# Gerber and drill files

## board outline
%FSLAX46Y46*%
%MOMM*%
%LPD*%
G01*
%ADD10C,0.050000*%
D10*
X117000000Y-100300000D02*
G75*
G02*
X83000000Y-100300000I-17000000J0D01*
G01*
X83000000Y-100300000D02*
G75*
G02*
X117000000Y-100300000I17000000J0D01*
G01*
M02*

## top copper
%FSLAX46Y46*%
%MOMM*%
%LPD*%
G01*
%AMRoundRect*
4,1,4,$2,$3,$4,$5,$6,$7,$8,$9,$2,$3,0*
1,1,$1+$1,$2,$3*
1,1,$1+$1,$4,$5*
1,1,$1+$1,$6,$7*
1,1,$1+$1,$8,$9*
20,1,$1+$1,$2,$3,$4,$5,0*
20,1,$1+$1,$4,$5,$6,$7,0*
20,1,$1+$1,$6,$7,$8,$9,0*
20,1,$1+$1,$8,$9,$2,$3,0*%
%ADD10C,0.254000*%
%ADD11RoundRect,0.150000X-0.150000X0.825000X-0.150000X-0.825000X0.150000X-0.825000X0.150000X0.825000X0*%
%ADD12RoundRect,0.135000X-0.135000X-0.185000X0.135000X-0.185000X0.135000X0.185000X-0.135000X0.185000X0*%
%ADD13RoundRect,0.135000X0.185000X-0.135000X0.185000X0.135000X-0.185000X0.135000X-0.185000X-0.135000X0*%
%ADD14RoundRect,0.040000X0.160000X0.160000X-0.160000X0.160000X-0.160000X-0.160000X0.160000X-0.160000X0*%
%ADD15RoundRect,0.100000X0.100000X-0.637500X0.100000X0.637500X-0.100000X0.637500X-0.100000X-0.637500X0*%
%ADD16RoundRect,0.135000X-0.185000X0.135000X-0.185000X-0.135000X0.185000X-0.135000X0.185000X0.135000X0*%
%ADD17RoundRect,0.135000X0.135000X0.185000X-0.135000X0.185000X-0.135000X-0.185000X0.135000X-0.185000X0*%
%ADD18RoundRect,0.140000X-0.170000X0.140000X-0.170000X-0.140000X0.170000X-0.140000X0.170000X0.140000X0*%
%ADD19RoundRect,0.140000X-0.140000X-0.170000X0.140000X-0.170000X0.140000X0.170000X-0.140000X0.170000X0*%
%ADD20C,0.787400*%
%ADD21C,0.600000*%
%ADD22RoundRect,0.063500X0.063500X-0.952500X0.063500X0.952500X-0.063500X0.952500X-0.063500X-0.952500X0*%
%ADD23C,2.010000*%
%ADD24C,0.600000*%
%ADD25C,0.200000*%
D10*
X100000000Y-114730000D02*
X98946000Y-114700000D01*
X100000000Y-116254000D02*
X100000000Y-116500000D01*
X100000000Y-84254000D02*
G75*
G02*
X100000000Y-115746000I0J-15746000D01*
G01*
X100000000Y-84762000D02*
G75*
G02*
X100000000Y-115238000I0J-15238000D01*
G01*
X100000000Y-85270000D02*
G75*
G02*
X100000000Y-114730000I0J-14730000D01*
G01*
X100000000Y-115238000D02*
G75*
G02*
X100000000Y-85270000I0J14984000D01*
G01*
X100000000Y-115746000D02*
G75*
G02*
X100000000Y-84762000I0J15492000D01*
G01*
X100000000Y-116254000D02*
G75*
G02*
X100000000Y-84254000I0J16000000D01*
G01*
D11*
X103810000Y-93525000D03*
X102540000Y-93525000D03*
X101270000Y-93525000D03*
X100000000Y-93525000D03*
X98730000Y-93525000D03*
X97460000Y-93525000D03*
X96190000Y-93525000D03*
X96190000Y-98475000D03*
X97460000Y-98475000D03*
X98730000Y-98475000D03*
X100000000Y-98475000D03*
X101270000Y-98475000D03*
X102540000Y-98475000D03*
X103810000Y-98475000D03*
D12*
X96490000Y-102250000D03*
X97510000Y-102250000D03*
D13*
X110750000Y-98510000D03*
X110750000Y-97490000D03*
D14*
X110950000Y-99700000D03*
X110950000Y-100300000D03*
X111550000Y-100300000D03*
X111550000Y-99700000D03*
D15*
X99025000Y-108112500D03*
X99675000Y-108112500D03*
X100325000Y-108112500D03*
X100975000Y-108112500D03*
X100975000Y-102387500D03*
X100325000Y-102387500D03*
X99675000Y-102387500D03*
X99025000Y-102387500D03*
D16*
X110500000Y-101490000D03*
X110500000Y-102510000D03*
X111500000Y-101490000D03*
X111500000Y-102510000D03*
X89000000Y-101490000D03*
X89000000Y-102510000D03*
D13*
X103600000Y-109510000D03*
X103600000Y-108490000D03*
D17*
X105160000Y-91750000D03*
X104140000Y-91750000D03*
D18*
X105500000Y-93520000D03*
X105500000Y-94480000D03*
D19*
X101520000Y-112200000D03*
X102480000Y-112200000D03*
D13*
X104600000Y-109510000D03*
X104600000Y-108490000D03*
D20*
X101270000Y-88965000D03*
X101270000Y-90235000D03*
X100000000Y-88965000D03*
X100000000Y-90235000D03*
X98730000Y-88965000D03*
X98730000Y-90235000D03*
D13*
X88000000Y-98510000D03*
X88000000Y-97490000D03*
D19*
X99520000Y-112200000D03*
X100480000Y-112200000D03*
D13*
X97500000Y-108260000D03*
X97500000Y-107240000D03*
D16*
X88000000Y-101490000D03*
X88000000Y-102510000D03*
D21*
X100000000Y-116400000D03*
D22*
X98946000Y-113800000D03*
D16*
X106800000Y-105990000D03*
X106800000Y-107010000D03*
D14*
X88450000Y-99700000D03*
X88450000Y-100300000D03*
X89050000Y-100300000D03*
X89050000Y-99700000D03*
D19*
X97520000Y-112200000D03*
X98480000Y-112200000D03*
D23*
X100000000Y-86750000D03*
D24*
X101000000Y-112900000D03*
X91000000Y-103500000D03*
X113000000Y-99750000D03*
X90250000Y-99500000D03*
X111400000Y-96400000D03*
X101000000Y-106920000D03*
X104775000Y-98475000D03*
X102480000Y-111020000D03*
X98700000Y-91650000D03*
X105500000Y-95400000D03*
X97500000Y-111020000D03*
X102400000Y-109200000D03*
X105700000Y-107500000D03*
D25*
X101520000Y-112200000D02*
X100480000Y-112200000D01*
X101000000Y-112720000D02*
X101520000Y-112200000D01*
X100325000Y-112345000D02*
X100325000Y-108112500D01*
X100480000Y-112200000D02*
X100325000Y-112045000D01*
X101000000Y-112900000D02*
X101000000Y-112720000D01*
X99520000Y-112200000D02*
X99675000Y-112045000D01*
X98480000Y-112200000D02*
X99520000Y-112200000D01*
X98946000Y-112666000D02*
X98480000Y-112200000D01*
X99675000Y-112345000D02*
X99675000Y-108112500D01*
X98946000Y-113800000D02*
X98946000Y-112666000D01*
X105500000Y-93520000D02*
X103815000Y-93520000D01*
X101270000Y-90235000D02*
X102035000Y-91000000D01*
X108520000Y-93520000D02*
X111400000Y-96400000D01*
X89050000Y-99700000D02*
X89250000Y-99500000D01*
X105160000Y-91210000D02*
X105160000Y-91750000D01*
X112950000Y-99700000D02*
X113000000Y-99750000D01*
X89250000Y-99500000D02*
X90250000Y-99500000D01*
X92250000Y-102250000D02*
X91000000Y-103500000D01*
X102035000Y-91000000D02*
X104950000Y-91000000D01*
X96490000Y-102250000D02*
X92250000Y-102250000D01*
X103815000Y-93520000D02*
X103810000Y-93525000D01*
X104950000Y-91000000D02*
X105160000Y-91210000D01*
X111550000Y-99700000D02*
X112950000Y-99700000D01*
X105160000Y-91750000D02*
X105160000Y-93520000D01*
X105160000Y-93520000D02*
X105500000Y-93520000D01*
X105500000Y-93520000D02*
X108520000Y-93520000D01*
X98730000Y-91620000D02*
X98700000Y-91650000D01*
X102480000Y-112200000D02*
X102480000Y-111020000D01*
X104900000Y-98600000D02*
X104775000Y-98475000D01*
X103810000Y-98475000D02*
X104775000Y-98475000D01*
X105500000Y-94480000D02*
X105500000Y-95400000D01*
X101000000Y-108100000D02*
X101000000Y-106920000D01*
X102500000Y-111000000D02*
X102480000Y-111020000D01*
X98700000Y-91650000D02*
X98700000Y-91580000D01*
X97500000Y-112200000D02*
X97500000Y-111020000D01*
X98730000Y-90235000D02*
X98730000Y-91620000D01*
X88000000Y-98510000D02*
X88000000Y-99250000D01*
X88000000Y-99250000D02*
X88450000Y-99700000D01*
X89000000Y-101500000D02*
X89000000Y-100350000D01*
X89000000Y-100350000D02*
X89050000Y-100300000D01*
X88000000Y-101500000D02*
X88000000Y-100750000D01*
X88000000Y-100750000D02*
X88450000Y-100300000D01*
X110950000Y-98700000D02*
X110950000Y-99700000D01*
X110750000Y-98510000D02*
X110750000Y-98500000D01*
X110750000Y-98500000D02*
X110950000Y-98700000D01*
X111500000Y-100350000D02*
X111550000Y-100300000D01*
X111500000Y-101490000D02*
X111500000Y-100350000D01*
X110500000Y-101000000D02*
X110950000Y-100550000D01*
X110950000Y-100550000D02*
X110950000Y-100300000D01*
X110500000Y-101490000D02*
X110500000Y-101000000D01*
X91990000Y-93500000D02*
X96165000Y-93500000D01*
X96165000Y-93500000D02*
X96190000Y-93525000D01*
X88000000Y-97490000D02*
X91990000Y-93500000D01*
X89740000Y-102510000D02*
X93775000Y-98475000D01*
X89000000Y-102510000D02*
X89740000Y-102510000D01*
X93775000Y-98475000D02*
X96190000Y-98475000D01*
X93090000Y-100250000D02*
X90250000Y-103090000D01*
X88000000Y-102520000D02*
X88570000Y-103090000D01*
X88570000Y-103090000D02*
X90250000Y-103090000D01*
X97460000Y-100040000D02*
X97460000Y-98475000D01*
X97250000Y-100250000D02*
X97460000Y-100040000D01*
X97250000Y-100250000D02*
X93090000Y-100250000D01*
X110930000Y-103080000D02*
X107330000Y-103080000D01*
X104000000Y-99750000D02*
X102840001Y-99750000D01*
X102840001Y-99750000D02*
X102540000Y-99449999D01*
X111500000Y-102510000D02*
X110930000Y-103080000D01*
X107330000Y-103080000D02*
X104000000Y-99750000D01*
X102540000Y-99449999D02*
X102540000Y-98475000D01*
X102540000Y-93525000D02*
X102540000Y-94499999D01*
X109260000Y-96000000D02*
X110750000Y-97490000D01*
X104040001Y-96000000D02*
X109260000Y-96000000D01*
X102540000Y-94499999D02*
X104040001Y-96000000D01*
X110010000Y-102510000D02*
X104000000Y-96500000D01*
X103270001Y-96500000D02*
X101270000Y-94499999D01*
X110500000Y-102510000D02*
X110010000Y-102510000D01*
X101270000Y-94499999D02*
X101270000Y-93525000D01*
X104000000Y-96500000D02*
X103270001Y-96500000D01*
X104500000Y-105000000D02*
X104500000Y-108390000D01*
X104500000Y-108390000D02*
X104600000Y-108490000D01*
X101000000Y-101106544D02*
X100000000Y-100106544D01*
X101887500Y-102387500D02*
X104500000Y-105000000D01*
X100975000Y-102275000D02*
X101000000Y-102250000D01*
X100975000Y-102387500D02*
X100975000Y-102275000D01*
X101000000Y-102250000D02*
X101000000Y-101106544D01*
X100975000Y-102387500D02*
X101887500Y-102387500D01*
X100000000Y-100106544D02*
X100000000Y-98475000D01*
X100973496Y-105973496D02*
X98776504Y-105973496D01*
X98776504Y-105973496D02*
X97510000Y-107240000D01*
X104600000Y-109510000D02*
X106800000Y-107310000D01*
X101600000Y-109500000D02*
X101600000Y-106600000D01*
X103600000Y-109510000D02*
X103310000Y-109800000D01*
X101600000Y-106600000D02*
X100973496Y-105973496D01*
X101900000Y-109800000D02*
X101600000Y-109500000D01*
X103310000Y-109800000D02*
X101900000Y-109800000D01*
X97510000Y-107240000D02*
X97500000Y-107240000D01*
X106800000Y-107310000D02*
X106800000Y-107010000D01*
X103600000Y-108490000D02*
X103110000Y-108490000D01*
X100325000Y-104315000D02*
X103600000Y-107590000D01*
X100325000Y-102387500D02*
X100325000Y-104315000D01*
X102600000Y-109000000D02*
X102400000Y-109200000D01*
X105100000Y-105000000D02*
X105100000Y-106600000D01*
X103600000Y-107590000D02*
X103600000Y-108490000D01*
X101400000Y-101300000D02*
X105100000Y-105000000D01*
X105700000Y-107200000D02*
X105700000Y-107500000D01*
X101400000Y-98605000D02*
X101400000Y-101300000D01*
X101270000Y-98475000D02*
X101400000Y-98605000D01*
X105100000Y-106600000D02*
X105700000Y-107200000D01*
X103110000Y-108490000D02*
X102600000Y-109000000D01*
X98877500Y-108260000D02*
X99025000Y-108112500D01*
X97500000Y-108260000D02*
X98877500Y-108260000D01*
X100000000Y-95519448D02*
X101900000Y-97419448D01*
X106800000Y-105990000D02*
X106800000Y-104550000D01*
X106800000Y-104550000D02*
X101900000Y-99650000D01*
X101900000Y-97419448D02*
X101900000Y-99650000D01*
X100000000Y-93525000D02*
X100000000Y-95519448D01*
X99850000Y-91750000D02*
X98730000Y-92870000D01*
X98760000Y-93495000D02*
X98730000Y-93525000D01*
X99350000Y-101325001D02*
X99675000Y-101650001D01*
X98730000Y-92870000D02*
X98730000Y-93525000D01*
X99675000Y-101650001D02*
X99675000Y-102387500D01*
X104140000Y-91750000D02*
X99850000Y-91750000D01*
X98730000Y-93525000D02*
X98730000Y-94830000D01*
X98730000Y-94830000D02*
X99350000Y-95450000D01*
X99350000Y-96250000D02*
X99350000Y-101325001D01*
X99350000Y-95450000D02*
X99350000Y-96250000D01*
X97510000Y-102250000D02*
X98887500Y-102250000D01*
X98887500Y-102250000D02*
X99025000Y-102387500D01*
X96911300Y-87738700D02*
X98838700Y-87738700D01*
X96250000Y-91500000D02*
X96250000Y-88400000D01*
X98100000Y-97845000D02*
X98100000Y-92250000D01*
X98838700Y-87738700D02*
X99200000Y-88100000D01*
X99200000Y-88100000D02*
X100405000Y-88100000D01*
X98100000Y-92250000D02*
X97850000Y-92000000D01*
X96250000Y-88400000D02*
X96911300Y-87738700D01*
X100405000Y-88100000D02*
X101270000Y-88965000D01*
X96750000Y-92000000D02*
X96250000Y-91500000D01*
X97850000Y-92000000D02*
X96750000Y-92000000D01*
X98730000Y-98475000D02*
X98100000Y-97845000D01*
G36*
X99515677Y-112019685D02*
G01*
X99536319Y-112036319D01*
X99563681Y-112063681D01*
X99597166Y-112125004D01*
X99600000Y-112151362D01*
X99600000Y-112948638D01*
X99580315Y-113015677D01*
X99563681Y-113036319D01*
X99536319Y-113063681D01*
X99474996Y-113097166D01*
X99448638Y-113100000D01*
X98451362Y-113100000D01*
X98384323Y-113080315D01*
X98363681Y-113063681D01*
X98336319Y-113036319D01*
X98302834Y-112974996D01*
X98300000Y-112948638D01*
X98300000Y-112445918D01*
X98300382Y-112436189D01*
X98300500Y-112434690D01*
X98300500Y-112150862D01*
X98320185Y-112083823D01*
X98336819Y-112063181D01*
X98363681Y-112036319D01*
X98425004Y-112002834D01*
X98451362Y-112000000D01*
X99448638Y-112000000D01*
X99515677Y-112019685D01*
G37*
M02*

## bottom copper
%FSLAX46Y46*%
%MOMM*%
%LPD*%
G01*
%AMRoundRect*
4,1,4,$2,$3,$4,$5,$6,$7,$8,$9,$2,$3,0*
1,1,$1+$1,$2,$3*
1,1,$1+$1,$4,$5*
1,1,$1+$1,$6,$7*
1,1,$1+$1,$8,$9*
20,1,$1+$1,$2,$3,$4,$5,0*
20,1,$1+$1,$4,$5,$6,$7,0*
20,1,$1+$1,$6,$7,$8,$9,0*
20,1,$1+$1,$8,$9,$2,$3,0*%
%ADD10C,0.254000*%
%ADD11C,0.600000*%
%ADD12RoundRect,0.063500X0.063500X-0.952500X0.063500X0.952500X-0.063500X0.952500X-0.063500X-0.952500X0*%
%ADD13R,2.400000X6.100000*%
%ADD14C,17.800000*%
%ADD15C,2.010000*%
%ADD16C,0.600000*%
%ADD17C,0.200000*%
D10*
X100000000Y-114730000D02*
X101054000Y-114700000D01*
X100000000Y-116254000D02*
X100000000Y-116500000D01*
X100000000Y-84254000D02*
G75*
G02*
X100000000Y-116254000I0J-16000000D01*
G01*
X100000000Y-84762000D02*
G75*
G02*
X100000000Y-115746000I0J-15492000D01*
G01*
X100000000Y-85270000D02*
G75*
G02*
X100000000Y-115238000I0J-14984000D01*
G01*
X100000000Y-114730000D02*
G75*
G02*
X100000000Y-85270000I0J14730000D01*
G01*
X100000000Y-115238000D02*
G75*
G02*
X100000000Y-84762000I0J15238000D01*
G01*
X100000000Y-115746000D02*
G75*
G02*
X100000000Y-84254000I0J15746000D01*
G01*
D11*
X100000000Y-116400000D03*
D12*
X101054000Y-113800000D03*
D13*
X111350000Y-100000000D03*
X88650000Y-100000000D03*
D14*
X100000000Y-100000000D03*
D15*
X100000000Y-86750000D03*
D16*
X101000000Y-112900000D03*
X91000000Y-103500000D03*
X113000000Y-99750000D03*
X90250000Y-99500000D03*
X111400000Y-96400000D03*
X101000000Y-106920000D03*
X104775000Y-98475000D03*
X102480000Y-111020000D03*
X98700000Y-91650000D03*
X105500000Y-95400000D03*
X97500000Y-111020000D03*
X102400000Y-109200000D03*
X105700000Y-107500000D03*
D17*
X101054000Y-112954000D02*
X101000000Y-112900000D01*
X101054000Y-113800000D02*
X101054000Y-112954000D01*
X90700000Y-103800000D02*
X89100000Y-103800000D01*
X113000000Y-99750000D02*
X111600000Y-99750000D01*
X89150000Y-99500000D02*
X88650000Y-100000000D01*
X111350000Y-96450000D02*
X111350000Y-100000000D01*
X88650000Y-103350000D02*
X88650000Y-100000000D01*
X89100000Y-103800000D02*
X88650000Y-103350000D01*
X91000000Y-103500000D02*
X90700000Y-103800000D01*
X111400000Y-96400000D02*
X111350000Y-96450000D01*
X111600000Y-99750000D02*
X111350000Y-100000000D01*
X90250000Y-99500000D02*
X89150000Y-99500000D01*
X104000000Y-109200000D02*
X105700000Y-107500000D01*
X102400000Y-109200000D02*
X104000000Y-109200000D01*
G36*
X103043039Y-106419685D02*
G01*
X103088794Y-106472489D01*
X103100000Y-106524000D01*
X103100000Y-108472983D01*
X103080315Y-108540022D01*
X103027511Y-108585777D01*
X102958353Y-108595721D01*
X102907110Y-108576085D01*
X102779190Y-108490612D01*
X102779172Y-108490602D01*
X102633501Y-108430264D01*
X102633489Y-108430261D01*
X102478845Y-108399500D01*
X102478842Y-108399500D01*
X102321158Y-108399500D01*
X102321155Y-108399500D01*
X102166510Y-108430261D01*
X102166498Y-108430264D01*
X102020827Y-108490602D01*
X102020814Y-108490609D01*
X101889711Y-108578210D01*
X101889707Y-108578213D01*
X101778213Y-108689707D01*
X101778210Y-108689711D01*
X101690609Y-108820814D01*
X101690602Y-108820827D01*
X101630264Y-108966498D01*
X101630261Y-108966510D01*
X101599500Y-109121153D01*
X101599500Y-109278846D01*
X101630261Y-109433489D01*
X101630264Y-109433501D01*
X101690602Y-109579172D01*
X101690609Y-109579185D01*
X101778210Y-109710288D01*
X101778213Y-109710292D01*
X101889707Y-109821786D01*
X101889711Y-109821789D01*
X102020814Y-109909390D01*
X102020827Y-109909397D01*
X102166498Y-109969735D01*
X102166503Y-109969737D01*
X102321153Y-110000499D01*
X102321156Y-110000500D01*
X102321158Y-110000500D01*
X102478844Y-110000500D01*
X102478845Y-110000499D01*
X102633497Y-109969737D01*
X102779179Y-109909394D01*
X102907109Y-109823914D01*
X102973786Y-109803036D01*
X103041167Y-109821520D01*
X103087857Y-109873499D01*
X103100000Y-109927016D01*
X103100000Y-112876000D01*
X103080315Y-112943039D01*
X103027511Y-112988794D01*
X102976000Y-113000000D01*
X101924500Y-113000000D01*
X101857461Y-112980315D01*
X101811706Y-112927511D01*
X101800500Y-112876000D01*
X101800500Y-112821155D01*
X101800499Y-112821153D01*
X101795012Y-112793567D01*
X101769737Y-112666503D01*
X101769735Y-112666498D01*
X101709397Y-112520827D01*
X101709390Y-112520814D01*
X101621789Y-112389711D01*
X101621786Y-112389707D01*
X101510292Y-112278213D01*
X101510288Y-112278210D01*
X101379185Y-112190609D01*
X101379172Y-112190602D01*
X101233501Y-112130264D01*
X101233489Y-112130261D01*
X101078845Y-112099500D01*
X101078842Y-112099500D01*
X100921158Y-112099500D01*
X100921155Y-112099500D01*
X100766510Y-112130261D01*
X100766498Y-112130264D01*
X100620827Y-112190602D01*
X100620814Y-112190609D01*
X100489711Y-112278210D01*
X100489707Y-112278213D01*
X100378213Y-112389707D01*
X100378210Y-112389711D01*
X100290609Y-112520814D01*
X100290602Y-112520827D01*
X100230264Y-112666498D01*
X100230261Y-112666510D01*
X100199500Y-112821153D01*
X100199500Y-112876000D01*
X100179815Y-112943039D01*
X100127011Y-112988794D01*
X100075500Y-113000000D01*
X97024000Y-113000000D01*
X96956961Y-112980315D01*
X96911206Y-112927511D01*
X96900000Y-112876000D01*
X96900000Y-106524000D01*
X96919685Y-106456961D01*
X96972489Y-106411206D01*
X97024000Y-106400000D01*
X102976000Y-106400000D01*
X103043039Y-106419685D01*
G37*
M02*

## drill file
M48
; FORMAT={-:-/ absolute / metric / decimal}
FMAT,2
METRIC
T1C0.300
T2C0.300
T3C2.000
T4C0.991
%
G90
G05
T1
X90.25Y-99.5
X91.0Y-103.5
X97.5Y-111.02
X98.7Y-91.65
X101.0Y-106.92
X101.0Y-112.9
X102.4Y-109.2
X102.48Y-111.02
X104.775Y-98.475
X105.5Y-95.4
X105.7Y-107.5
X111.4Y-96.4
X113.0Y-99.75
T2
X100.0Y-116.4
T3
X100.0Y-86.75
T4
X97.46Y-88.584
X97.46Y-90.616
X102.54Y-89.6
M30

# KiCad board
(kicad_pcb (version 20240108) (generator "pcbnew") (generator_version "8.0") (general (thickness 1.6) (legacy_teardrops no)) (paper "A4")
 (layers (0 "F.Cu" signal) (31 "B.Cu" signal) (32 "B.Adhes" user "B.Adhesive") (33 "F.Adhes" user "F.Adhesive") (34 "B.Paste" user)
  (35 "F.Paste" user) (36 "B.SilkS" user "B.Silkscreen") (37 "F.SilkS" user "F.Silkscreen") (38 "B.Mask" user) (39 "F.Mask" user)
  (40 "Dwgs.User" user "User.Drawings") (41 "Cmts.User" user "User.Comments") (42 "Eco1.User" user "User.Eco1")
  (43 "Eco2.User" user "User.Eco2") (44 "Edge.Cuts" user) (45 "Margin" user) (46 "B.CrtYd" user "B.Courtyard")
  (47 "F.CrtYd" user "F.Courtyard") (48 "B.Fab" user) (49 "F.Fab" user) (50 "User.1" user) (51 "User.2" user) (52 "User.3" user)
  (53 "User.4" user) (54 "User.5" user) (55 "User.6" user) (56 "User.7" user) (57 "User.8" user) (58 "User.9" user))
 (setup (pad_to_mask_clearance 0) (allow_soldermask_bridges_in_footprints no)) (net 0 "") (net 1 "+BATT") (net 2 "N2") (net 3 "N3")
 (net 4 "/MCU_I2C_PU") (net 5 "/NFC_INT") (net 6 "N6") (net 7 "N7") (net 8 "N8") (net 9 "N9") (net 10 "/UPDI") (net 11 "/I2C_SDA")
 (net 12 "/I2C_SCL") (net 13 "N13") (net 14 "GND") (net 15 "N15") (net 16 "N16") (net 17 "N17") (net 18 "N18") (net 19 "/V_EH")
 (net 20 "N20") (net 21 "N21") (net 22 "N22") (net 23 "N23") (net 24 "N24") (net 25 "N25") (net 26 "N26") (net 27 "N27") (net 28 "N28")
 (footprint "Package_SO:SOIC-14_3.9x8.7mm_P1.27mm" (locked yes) (layer "F.Cu") (at 100 96 -90)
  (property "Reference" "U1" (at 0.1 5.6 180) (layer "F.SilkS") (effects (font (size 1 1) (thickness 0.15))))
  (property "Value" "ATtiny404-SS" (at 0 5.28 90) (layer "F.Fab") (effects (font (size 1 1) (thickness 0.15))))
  (pad "1" smd roundrect (at -2.475 -3.81 270) (size 1.95 0.6) (layers "F.Cu" "F.Paste" "F.Mask") (roundrect_rratio 0.25) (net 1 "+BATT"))
  (pad "2" smd roundrect (at -2.475 -2.54 270) (size 1.95 0.6) (layers "F.Cu" "F.Paste" "F.Mask") (roundrect_rratio 0.25) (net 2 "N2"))
  (pad "3" smd roundrect (at -2.475 -1.27 270) (size 1.95 0.6) (layers "F.Cu" "F.Paste" "F.Mask") (roundrect_rratio 0.25) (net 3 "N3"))
  (pad "4" smd roundrect (at -2.475 0 270) (size 1.95 0.6) (layers "F.Cu" "F.Paste" "F.Mask") (roundrect_rratio 0.25) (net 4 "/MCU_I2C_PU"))
  (pad "5" smd roundrect (at -2.475 1.27 270) (size 1.95 0.6) (layers "F.Cu" "F.Paste" "F.Mask") (roundrect_rratio 0.25) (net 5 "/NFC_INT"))
  (pad "6" smd roundrect (at -2.475 2.54 270) (size 1.95 0.6) (layers "F.Cu" "F.Paste" "F.Mask") (roundrect_rratio 0.25) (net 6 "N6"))
  (pad "7" smd roundrect (at -2.475 3.81 270) (size 1.95 0.6) (layers "F.Cu" "F.Paste" "F.Mask") (roundrect_rratio 0.25) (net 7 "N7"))
  (pad "8" smd roundrect (at 2.475 3.81 270) (size 1.95 0.6) (layers "F.Cu" "F.Paste" "F.Mask") (roundrect_rratio 0.25) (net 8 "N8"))
  (pad "9" smd roundrect (at 2.475 2.54 270) (size 1.95 0.6) (layers "F.Cu" "F.Paste" "F.Mask") (roundrect_rratio 0.25) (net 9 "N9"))
  (pad "10" smd roundrect (at 2.475 1.27 270) (size 1.95 0.6) (layers "F.Cu" "F.Paste" "F.Mask") (roundrect_rratio 0.25) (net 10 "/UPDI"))
  (pad "11" smd roundrect (at 2.475 0 270) (size 1.95 0.6) (layers "F.Cu" "F.Paste" "F.Mask") (roundrect_rratio 0.25) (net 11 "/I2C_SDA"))
  (pad "12" smd roundrect (at 2.475 -1.27 270) (size 1.95 0.6) (layers "F.Cu" "F.Paste" "F.Mask") (roundrect_rratio 0.25)
   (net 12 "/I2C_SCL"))
  (pad "13" smd roundrect (at 2.475 -2.54 270) (size 1.95 0.6) (layers "F.Cu" "F.Paste" "F.Mask") (roundrect_rratio 0.25) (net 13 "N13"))
  (pad "14" smd roundrect (at 2.475 -3.81 270) (size 1.95 0.6) (layers "F.Cu" "F.Paste" "F.Mask") (roundrect_rratio 0.25) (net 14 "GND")))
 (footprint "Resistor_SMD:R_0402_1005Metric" (layer "F.Cu") (at 97 102.25)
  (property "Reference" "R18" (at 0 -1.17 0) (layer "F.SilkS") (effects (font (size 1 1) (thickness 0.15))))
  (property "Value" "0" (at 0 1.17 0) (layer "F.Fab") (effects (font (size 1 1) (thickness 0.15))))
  (pad "1" smd roundrect (at -0.51 0) (size 0.54 0.64) (layers "F.Cu" "F.Paste" "F.Mask") (roundrect_rratio 0.25) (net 1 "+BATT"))
  (pad "2" smd roundrect (at 0.51 0) (size 0.54 0.64) (layers "F.Cu" "F.Paste" "F.Mask") (roundrect_rratio 0.25) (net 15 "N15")))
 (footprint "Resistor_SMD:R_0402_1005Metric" (layer "F.Cu") (at 110.75 98 90)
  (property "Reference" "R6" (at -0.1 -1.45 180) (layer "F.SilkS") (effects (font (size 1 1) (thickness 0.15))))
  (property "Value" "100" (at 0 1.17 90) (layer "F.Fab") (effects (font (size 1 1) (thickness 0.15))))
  (pad "1" smd roundrect (at -0.51 0 90) (size 0.54 0.64) (layers "F.Cu" "F.Paste" "F.Mask") (roundrect_rratio 0.25) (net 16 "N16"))
  (pad "2" smd roundrect (at 0.51 0 90) (size 0.54 0.64) (layers "F.Cu" "F.Paste" "F.Mask") (roundrect_rratio 0.25) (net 2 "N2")))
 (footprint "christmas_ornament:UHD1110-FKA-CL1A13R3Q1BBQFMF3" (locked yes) (layer "F.Cu") (at 111.25 100)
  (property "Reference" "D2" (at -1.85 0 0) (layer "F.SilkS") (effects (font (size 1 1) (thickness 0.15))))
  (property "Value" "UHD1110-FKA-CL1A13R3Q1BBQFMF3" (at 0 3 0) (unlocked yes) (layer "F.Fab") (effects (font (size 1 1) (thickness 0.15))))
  (pad "1" smd roundrect (at -0.3 -0.3 180) (size 0.4 0.4) (layers "F.Cu" "F.Paste" "F.Mask") (roundrect_rratio 0.1) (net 16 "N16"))
  (pad "2" smd roundrect (at -0.3 0.3 180) (size 0.4 0.4) (layers "F.Cu" "F.Paste" "F.Mask") (roundrect_rratio 0.1) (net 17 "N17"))
  (pad "3" smd roundrect (at 0.3 0.3 180) (size 0.4 0.4) (layers "F.Cu" "F.Paste" "F.Mask") (roundrect_rratio 0.1) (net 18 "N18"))
  (pad "4" smd roundrect (at 0.3 -0.3 180) (size 0.4 0.4) (layers "F.Cu" "F.Paste" "F.Mask") (roundrect_rratio 0.1) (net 1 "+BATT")))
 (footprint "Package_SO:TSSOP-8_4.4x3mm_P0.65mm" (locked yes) (layer "F.Cu") (at 100 105.25 90)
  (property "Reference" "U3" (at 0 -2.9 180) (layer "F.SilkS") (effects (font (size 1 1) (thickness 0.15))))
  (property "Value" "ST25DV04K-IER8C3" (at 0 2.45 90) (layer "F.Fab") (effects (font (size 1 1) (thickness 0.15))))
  (pad "1" smd roundrect (at -2.8625 -0.975 90) (size 1.475 0.4) (layers "F.Cu" "F.Paste" "F.Mask") (roundrect_rratio 0.25) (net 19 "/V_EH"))
  (pad "2" smd roundrect (at -2.8625 -0.325 90) (size 1.475 0.4) (layers "F.Cu" "F.Paste" "F.Mask") (roundrect_rratio 0.25) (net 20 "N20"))
  (pad "3" smd roundrect (at -2.8625 0.325 90) (size 1.475 0.4) (layers "F.Cu" "F.Paste" "F.Mask") (roundrect_rratio 0.25) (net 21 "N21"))
  (pad "4" smd roundrect (at -2.8625 0.975 90) (size 1.475 0.4) (layers "F.Cu" "F.Paste" "F.Mask") (roundrect_rratio 0.25) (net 14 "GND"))
  (pad "5" smd roundrect (at 2.8625 0.975 90) (size 1.475 0.4) (layers "F.Cu" "F.Paste" "F.Mask") (roundrect_rratio 0.25)
   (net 11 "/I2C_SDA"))
  (pad "6" smd roundrect (at 2.8625 0.325 90) (size 1.475 0.4) (layers "F.Cu" "F.Paste" "F.Mask") (roundrect_rratio 0.25)
   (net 12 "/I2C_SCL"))
  (pad "7" smd roundrect (at 2.8625 -0.325 90) (size 1.475 0.4) (layers "F.Cu" "F.Paste" "F.Mask") (roundrect_rratio 0.25)
   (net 5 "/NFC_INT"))
  (pad "8" smd roundrect (at 2.8625 -0.975 90) (size 1.475 0.4) (layers "F.Cu" "F.Paste" "F.Mask") (roundrect_rratio 0.25) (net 15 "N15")))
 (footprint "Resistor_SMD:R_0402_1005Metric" (layer "F.Cu") (at 110.5 102 -90)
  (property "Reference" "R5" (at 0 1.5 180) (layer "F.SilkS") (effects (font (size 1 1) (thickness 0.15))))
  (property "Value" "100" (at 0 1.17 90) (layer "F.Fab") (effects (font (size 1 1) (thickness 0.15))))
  (pad "1" smd roundrect (at -0.51 0 270) (size 0.54 0.64) (layers "F.Cu" "F.Paste" "F.Mask") (roundrect_rratio 0.25) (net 17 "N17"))
  (pad "2" smd roundrect (at 0.51 0 270) (size 0.54 0.64) (layers "F.Cu" "F.Paste" "F.Mask") (roundrect_rratio 0.25) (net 3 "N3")))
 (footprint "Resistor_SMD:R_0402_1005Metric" (layer "F.Cu") (at 111.5 102 -90)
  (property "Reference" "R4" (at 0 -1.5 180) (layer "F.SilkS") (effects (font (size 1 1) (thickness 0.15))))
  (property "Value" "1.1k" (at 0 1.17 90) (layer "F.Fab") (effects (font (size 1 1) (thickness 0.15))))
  (pad "1" smd roundrect (at -0.51 0 270) (size 0.54 0.64) (layers "F.Cu" "F.Paste" "F.Mask") (roundrect_rratio 0.25) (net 18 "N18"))
  (pad "2" smd roundrect (at 0.51 0 270) (size 0.54 0.64) (layers "F.Cu" "F.Paste" "F.Mask") (roundrect_rratio 0.25) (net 13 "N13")))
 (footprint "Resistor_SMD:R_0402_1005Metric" (layer "F.Cu") (at 89 102 -90)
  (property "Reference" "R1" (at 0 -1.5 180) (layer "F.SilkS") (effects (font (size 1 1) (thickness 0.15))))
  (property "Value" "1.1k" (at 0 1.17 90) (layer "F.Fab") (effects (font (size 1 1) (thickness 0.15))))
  (pad "1" smd roundrect (at -0.51 0 270) (size 0.54 0.64) (layers "F.Cu" "F.Paste" "F.Mask") (roundrect_rratio 0.25) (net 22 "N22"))
  (pad "2" smd roundrect (at 0.51 0 270) (size 0.54 0.64) (layers "F.Cu" "F.Paste" "F.Mask") (roundrect_rratio 0.25) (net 8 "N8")))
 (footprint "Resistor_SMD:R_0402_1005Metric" (layer "F.Cu") (at 103.6 109 90)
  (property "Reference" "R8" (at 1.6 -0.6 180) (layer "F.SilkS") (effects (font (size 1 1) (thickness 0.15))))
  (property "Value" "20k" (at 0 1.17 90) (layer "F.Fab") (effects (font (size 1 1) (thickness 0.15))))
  (pad "1" smd roundrect (at -0.51 0 90) (size 0.54 0.64) (layers "F.Cu" "F.Paste" "F.Mask") (roundrect_rratio 0.25) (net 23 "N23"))
  (pad "2" smd roundrect (at 0.51 0 90) (size 0.54 0.64) (layers "F.Cu" "F.Paste" "F.Mask") (roundrect_rratio 0.25) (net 12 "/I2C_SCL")))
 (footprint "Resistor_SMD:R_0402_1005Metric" (layer "F.Cu") (at 104.65 91.75 180)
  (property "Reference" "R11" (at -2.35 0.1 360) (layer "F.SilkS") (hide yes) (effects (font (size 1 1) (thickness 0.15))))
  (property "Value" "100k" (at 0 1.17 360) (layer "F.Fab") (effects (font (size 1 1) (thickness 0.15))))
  (pad "1" smd roundrect (at -0.51 0 180) (size 0.54 0.64) (layers "F.Cu" "F.Paste" "F.Mask") (roundrect_rratio 0.25) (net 1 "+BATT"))
  (pad "2" smd roundrect (at 0.51 0 180) (size 0.54 0.64) (layers "F.Cu" "F.Paste" "F.Mask") (roundrect_rratio 0.25) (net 5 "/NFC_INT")))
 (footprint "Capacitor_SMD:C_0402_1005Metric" (layer "F.Cu") (at 105.5 94 -90)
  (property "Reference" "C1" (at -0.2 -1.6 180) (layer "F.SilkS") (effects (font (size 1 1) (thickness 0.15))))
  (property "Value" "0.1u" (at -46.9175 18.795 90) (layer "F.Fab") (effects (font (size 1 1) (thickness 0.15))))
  (pad "1" smd roundrect (at -0.48 0 270) (size 0.56 0.62) (layers "F.Cu" "F.Paste" "F.Mask") (roundrect_rratio 0.25) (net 1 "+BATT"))
  (pad "2" smd roundrect (at 0.48 0 270) (size 0.56 0.62) (layers "F.Cu" "F.Paste" "F.Mask") (roundrect_rratio 0.25) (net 14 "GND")))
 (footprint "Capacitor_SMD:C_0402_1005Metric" (layer "F.Cu") (at 102 112.2)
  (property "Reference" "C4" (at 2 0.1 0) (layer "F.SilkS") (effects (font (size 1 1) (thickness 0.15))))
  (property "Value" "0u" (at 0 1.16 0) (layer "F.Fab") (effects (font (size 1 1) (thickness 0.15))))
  (pad "1" smd roundrect (at -0.48 0) (size 0.56 0.62) (layers "F.Cu" "F.Paste" "F.Mask") (roundrect_rratio 0.25) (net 21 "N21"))
  (pad "2" smd roundrect (at 0.48 0) (size 0.56 0.62) (layers "F.Cu" "F.Paste" "F.Mask") (roundrect_rratio 0.25) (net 14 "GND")))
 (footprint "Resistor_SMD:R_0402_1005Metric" (layer "F.Cu") (at 104.6 109 90)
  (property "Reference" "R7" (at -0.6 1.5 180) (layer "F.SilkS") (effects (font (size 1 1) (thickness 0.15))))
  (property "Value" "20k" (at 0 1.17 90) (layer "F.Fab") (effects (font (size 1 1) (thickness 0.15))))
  (pad "1" smd roundrect (at -0.51 0 90) (size 0.54 0.64) (layers "F.Cu" "F.Paste" "F.Mask") (roundrect_rratio 0.25) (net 23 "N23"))
  (pad "2" smd roundrect (at 0.51 0 90) (size 0.54 0.64) (layers "F.Cu" "F.Paste" "F.Mask") (roundrect_rratio 0.25) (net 11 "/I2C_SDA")))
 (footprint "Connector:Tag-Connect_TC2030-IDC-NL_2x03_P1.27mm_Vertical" (layer "F.Cu") (at 100 89.6 180)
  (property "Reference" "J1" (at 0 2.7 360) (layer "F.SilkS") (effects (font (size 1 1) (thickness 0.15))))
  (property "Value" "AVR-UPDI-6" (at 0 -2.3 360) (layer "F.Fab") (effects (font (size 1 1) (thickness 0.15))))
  (pad "" np_thru_hole circle (at -2.54 0 180) (size 0.9906 0.9906) (drill 0.9906) (layers "*.Cu" "*.Mask"))
  (pad "" np_thru_hole circle (at 2.54 -1.016 180) (size 0.9906 0.9906) (drill 0.9906) (layers "*.Cu" "*.Mask"))
  (pad "" np_thru_hole circle (at 2.54 1.016 180) (size 0.9906 0.9906) (drill 0.9906) (layers "*.Cu" "*.Mask"))
  (pad "1" connect circle (at -1.27 0.635 180) (size 0.7874 0.7874) (layers "F.Cu" "F.Mask") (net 10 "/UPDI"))
  (pad "2" connect circle (at -1.27 -0.635 180) (size 0.7874 0.7874) (layers "F.Cu" "F.Mask") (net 1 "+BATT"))
  (pad "3" connect circle (at 0 0.635 180) (size 0.7874 0.7874) (layers "F.Cu" "F.Mask") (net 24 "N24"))
  (pad "4" connect circle (at 0 -0.635 180) (size 0.7874 0.7874) (layers "F.Cu" "F.Mask") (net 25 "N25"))
  (pad "5" connect circle (at 1.27 0.635 180) (size 0.7874 0.7874) (layers "F.Cu" "F.Mask") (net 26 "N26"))
  (pad "6" connect circle (at 1.27 -0.635 180) (size 0.7874 0.7874) (layers "F.Cu" "F.Mask") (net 14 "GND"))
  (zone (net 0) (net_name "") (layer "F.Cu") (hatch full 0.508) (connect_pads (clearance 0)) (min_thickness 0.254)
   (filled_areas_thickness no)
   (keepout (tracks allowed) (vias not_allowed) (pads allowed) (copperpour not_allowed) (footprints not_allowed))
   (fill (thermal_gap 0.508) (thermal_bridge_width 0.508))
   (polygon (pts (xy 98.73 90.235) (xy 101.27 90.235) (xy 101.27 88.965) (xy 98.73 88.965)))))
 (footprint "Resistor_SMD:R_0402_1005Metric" (layer "F.Cu") (at 88 98 90)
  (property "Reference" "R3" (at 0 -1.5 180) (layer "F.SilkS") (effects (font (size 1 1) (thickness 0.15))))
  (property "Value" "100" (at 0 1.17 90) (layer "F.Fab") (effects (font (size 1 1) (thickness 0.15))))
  (pad "1" smd roundrect (at -0.51 0 90) (size 0.54 0.64) (layers "F.Cu" "F.Paste" "F.Mask") (roundrect_rratio 0.25) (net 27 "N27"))
  (pad "2" smd roundrect (at 0.51 0 90) (size 0.54 0.64) (layers "F.Cu" "F.Paste" "F.Mask") (roundrect_rratio 0.25) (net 7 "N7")))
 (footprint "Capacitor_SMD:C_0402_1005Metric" (layer "F.Cu") (at 100 112.2)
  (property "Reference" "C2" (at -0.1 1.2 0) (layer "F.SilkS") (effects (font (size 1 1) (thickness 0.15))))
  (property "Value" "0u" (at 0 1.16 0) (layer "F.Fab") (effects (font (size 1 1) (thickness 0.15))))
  (pad "1" smd roundrect (at -0.48 0) (size 0.56 0.62) (layers "F.Cu" "F.Paste" "F.Mask") (roundrect_rratio 0.25) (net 20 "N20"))
  (pad "2" smd roundrect (at 0.48 0) (size 0.56 0.62) (layers "F.Cu" "F.Paste" "F.Mask") (roundrect_rratio 0.25) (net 21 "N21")))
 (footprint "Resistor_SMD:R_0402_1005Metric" (layer "F.Cu") (at 97.5 107.75 90)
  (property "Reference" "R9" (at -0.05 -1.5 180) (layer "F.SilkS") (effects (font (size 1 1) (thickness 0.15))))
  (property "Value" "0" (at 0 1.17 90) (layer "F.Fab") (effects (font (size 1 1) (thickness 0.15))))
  (pad "1" smd roundrect (at -0.51 0 90) (size 0.54 0.64) (layers "F.Cu" "F.Paste" "F.Mask") (roundrect_rratio 0.25) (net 19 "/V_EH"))
  (pad "2" smd roundrect (at 0.51 0 90) (size 0.54 0.64) (layers "F.Cu" "F.Paste" "F.Mask") (roundrect_rratio 0.25) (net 23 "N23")))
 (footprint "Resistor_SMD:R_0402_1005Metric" (layer "F.Cu") (at 88 102 -90)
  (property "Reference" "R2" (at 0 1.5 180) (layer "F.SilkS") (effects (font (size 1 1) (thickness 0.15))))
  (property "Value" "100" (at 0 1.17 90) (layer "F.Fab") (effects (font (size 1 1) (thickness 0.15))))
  (pad "1" smd roundrect (at -0.51 0 270) (size 0.54 0.64) (layers "F.Cu" "F.Paste" "F.Mask") (roundrect_rratio 0.25) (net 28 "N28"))
  (pad "2" smd roundrect (at 0.51 0 270) (size 0.54 0.64) (layers "F.Cu" "F.Paste" "F.Mask") (roundrect_rratio 0.25) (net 9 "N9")))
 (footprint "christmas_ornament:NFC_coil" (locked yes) (layer "F.Cu") (at 100 100 -90)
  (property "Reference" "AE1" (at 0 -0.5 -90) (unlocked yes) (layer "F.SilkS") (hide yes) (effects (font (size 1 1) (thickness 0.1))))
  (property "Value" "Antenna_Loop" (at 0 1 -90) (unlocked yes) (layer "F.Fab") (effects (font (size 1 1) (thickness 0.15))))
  (fp_line (start 14.73 0) (end 14.7 1.054) (stroke (width 0.254) (type default)) (layer "F.Cu"))
  (fp_line (start 16.254 0) (end 16.5 0) (stroke (width 0.254) (type default)) (layer "F.Cu"))
  (fp_arc (start -15.746 0) (mid 0 -15.746) (end 15.746 0) (stroke (width 0.254) (type default)) (layer "F.Cu"))
  (fp_arc (start -15.238 0) (mid 0 -15.238) (end 15.238 0) (stroke (width 0.254) (type default)) (layer "F.Cu"))
  (fp_arc (start -14.73 0) (mid 0 -14.73) (end 14.73 0) (stroke (width 0.254) (type default)) (layer "F.Cu"))
  (fp_arc (start 15.238 0) (mid 0.254 14.984) (end -14.73 0) (stroke (width 0.254) (type default)) (layer "F.Cu"))
  (fp_arc (start 15.746 0) (mid 0.254 15.492) (end -15.238 0) (stroke (width 0.254) (type default)) (layer "F.Cu"))
  (fp_arc (start 16.254 0) (mid 0.254 16) (end -15.746 0) (stroke (width 0.254) (type default)) (layer "F.Cu"))
  (fp_line (start 14.73 0) (end 14.7 -1.054) (stroke (width 0.254) (type default)) (layer "B.Cu"))
  (fp_line (start 16.254 0) (end 16.5 0) (stroke (width 0.254) (type default)) (layer "B.Cu"))
  (fp_arc (start -15.746 0) (mid 0.254 -16) (end 16.254 0) (stroke (width 0.254) (type default)) (layer "B.Cu"))
  (fp_arc (start -15.238 0) (mid 0.254 -15.492) (end 15.746 0) (stroke (width 0.254) (type default)) (layer "B.Cu"))
  (fp_arc (start -14.73 0) (mid 0.254 -14.984) (end 15.238 0) (stroke (width 0.254) (type default)) (layer "B.Cu"))
  (fp_arc (start 14.73 0) (mid 0 14.73) (end -14.73 0) (stroke (width 0.254) (type default)) (layer "B.Cu"))
  (fp_arc (start 15.238 0) (mid 0 15.238) (end -15.238 0) (stroke (width 0.254) (type default)) (layer "B.Cu"))
  (fp_arc (start 15.746 0) (mid 0 15.746) (end -15.746 0) (stroke (width 0.254) (type default)) (layer "B.Cu"))
  (pad "" thru_hole circle (at 16.4 0 90) (size 0.6 0.6) (drill 0.3) (layers "*.Cu") (remove_unused_layers yes) (keep_end_layers yes)
   (zone_layer_connections))
  (pad "1" smd roundrect (at 13.8 1.054 90) (size 2.032 0.254) (layers "F.Cu") (roundrect_rratio 0.25) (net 20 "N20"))
  (pad "2" smd roundrect (at 13.8 -1.054 90) (size 2.032 0.254) (layers "B.Cu") (roundrect_rratio 0.25) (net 21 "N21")))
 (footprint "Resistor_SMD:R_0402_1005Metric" (layer "F.Cu") (at 106.8 106.5 -90)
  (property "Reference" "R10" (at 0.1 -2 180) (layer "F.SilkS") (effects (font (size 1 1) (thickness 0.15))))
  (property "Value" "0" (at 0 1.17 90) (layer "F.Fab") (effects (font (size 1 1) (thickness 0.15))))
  (pad "1" smd roundrect (at -0.51 0 270) (size 0.54 0.64) (layers "F.Cu" "F.Paste" "F.Mask") (roundrect_rratio 0.25) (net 4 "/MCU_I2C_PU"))
  (pad "2" smd roundrect (at 0.51 0 270) (size 0.54 0.64) (layers "F.Cu" "F.Paste" "F.Mask") (roundrect_rratio 0.25) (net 23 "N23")))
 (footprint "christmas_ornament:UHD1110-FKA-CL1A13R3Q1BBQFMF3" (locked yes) (layer "F.Cu") (at 88.75 100)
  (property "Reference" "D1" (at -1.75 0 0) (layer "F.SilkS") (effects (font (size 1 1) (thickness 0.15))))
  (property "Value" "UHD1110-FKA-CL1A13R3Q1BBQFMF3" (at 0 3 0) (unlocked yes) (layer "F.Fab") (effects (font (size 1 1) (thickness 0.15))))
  (pad "1" smd roundrect (at -0.3 -0.3 180) (size 0.4 0.4) (layers "F.Cu" "F.Paste" "F.Mask") (roundrect_rratio 0.1) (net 27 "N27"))
  (pad "2" smd roundrect (at -0.3 0.3 180) (size 0.4 0.4) (layers "F.Cu" "F.Paste" "F.Mask") (roundrect_rratio 0.1) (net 28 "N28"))
  (pad "3" smd roundrect (at 0.3 0.3 180) (size 0.4 0.4) (layers "F.Cu" "F.Paste" "F.Mask") (roundrect_rratio 0.1) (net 22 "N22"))
  (pad "4" smd roundrect (at 0.3 -0.3 180) (size 0.4 0.4) (layers "F.Cu" "F.Paste" "F.Mask") (roundrect_rratio 0.1) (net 1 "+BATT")))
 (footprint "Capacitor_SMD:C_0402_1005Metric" (layer "F.Cu") (at 98 112.2)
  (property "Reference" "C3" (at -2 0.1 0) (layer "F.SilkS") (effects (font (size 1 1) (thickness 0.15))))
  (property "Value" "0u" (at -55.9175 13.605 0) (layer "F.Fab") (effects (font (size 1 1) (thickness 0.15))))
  (pad "1" smd roundrect (at -0.48 0) (size 0.56 0.62) (layers "F.Cu" "F.Paste" "F.Mask") (roundrect_rratio 0.25) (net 14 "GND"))
  (pad "2" smd roundrect (at 0.48 0) (size 0.56 0.62) (layers "F.Cu" "F.Paste" "F.Mask") (roundrect_rratio 0.25) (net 20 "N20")))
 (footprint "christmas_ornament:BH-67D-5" (layer "B.Cu") (at 100 100 180)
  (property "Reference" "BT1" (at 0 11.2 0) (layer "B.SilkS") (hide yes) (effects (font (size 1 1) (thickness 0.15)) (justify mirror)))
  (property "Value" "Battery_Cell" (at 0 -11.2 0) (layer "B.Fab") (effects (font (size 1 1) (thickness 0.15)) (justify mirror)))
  (pad "1" smd rect (at -11.35 0 180) (size 2.4 6.1) (layers "B.Cu" "B.Paste" "B.Mask") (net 1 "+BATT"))
  (pad "1" smd rect (at 11.35 0 180) (size 2.4 6.1) (layers "B.Cu" "B.Paste" "B.Mask") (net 1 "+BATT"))
  (pad "2" smd circle (at 0 0 180) (size 17.8 17.8) (layers "B.Cu" "B.Mask") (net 14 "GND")))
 (gr_circle (center 100 100.3) (end 117 100.3) (stroke (width 0.05) (type default)) (fill none) (layer "Edge.Cuts"))
 (via (at 100 86.75) (size 2.01) (drill 2) (layers "F.Cu" "B.Cu") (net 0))
 (segment (start 101.52 112.2) (end 100.48 112.2) (width 0.2) (layer "F.Cu") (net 21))
 (segment (start 101 112.72) (end 101.52 112.2) (width 0.2) (layer "F.Cu") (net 21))
 (segment (start 100.325 112.345) (end 100.325 108.1125) (width 0.2) (layer "F.Cu") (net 21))
 (segment (start 100.48 112.2) (end 100.325 112.045) (width 0.2) (layer "F.Cu") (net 21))
 (segment (start 101 112.9) (end 101 112.72) (width 0.2) (layer "F.Cu") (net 21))
 (via (at 101 112.9) (size 0.6) (drill 0.3) (layers "F.Cu" "B.Cu") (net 21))
 (segment (start 101.054 112.954) (end 101 112.9) (width 0.2) (layer "B.Cu") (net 21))
 (segment (start 101.054 113.8) (end 101.054 112.954) (width 0.2) (layer "B.Cu") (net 21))
 (segment (start 99.52 112.2) (end 99.675 112.045) (width 0.2) (layer "F.Cu") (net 20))
 (segment (start 98.48 112.2) (end 99.52 112.2) (width 0.2) (layer "F.Cu") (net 20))
 (segment (start 98.946 112.666) (end 98.48 112.2) (width 0.2) (layer "F.Cu") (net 20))
 (segment (start 99.675 112.345) (end 99.675 108.1125) (width 0.2) (layer "F.Cu") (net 20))
 (segment (start 98.946 113.8) (end 98.946 112.666) (width 0.2) (layer "F.Cu") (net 20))
 (segment (start 105.5 93.52) (end 103.815 93.52) (width 0.2) (layer "F.Cu") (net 1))
 (segment (start 101.27 90.235) (end 102.035 91) (width 0.2) (layer "F.Cu") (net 1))
 (segment (start 108.52 93.52) (end 111.4 96.4) (width 0.2) (layer "F.Cu") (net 1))
 (segment (start 89.05 99.7) (end 89.25 99.5) (width 0.2) (layer "F.Cu") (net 1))
 (segment (start 105.16 91.21) (end 105.16 91.75) (width 0.2) (layer "F.Cu") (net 1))
 (segment (start 112.95 99.7) (end 113 99.75) (width 0.2) (layer "F.Cu") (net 1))
 (segment (start 89.25 99.5) (end 90.25 99.5) (width 0.2) (layer "F.Cu") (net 1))
 (segment (start 92.25 102.25) (end 91 103.5) (width 0.2) (layer "F.Cu") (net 1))
 (segment (start 102.035 91) (end 104.95 91) (width 0.2) (layer "F.Cu") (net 1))
 (segment (start 96.49 102.25) (end 92.25 102.25) (width 0.2) (layer "F.Cu") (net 1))
 (segment (start 103.815 93.52) (end 103.81 93.525) (width 0.2) (layer "F.Cu") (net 1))
 (segment (start 104.95 91) (end 105.16 91.21) (width 0.2) (layer "F.Cu") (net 1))
 (segment (start 111.55 99.7) (end 112.95 99.7) (width 0.2) (layer "F.Cu") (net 1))
 (segment (start 105.16 91.75) (end 105.16 93.52) (width 0.2) (layer "F.Cu") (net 1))
 (segment (start 105.16 93.52) (end 105.5 93.52) (width 0.2) (layer "F.Cu") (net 1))
 (segment (start 105.5 93.52) (end 108.52 93.52) (width 0.2) (layer "F.Cu") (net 1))
 (via (at 91 103.5) (size 0.6) (drill 0.3) (layers "F.Cu" "B.Cu") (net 1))
 (via (at 113 99.75) (size 0.6) (drill 0.3) (layers "F.Cu" "B.Cu") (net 1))
 (via (at 90.25 99.5) (size 0.6) (drill 0.3) (layers "F.Cu" "B.Cu") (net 1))
 (via (at 111.4 96.4) (size 0.6) (drill 0.3) (layers "F.Cu" "B.Cu") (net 1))
 (segment (start 90.7 103.8) (end 89.1 103.8) (width 0.2) (layer "B.Cu") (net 1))
 (segment (start 113 99.75) (end 111.6 99.75) (width 0.2) (layer "B.Cu") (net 1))
 (segment (start 89.15 99.5) (end 88.65 100) (width 0.2) (layer "B.Cu") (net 1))
 (segment (start 111.35 96.45) (end 111.35 100) (width 0.2) (layer "B.Cu") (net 1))
 (segment (start 88.65 103.35) (end 88.65 100) (width 0.2) (layer "B.Cu") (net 1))
 (segment (start 89.1 103.8) (end 88.65 103.35) (width 0.2) (layer "B.Cu") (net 1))
 (segment (start 91 103.5) (end 90.7 103.8) (width 0.2) (layer "B.Cu") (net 1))
 (segment (start 111.4 96.4) (end 111.35 96.45) (width 0.2) (layer "B.Cu") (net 1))
 (segment (start 111.6 99.75) (end 111.35 100) (width 0.2) (layer "B.Cu") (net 1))
 (segment (start 90.25 99.5) (end 89.15 99.5) (width 0.2) (layer "B.Cu") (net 1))
 (segment (start 98.73 91.62) (end 98.7 91.65) (width 0.2) (layer "F.Cu") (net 14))
 (segment (start 102.48 112.2) (end 102.48 111.02) (width 0.2) (layer "F.Cu") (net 14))
 (segment (start 104.9 98.6) (end 104.775 98.475) (width 0.2) (layer "F.Cu") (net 14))
 (segment (start 103.81 98.475) (end 104.775 98.475) (width 0.2) (layer "F.Cu") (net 14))
 (segment (start 105.5 94.48) (end 105.5 95.4) (width 0.2) (layer "F.Cu") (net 14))
 (segment (start 101 108.1) (end 101 106.92) (width 0.2) (layer "F.Cu") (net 14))
 (segment (start 102.5 111) (end 102.48 111.02) (width 0.2) (layer "F.Cu") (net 14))
 (segment (start 98.7 91.65) (end 98.7 91.58) (width 0.2) (layer "F.Cu") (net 14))
 (segment (start 97.5 112.2) (end 97.5 111.02) (width 0.2) (layer "F.Cu") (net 14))
 (segment (start 98.73 90.235) (end 98.73 91.62) (width 0.2) (layer "F.Cu") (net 14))
 (via (at 101 106.92) (size 0.6) (drill 0.3) (layers "F.Cu" "B.Cu") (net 14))
 (via (at 104.775 98.475) (size 0.6) (drill 0.3) (layers "F.Cu" "B.Cu") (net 14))
 (via (at 102.48 111.02) (size 0.6) (drill 0.3) (layers "F.Cu" "B.Cu") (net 14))
 (via (at 98.7 91.65) (size 0.6) (drill 0.3) (layers "F.Cu" "B.Cu") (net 14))
 (via (at 105.5 95.4) (size 0.6) (drill 0.3) (layers "F.Cu" "B.Cu") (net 14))
 (via (at 97.5 111.02) (size 0.6) (drill 0.3) (layers "F.Cu" "B.Cu") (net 14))
 (segment (start 88 98.51) (end 88 99.25) (width 0.2) (layer "F.Cu") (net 27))
 (segment (start 88 99.25) (end 88.45 99.7) (width 0.2) (layer "F.Cu") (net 27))
 (segment (start 89 101.5) (end 89 100.35) (width 0.2) (layer "F.Cu") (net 22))
 (segment (start 89 100.35) (end 89.05 100.3) (width 0.2) (layer "F.Cu") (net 22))
 (segment (start 88 101.5) (end 88 100.75) (width 0.2) (layer "F.Cu") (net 28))
 (segment (start 88 100.75) (end 88.45 100.3) (width 0.2) (layer "F.Cu") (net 28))
 (segment (start 110.95 98.7) (end 110.95 99.7) (width 0.2) (layer "F.Cu") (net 16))
 (segment (start 110.75 98.51) (end 110.75 98.5) (width 0.2) (layer "F.Cu") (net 16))
 (segment (start 110.75 98.5) (end 110.95 98.7) (width 0.2) (layer "F.Cu") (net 16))
 (segment (start 111.5 100.35) (end 111.55 100.3) (width 0.2) (layer "F.Cu") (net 18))
 (segment (start 111.5 101.49) (end 111.5 100.35) (width 0.2) (layer "F.Cu") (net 18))
 (segment (start 110.5 101) (end 110.95 100.55) (width 0.2) (layer "F.Cu") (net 17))
 (segment (start 110.95 100.55) (end 110.95 100.3) (width 0.2) (layer "F.Cu") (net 17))
 (segment (start 110.5 101.49) (end 110.5 101) (width 0.2) (layer "F.Cu") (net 17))
 (segment (start 91.99 93.5) (end 96.165 93.5) (width 0.2) (layer "F.Cu") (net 7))
 (segment (start 96.165 93.5) (end 96.19 93.525) (width 0.2) (layer "F.Cu") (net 7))
 (segment (start 88 97.49) (end 91.99 93.5) (width 0.2) (layer "F.Cu") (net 7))
 (segment (start 89.74 102.51) (end 93.775 98.475) (width 0.2) (layer "F.Cu") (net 8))
 (segment (start 89 102.51) (end 89.74 102.51) (width 0.2) (layer "F.Cu") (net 8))
 (segment (start 93.775 98.475) (end 96.19 98.475) (width 0.2) (layer "F.Cu") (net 8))
 (segment (start 93.09 100.25) (end 90.25 103.09) (width 0.2) (layer "F.Cu") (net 9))
 (segment (start 88 102.52) (end 88.57 103.09) (width 0.2) (layer "F.Cu") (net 9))
 (segment (start 88.57 103.09) (end 90.25 103.09) (width 0.2) (layer "F.Cu") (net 9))
 (segment (start 97.46 100.04) (end 97.46 98.475) (width 0.2) (layer "F.Cu") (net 9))
 (segment (start 97.25 100.25) (end 97.46 100.04) (width 0.2) (layer "F.Cu") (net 9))
 (segment (start 97.25 100.25) (end 93.09 100.25) (width 0.2) (layer "F.Cu") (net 9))
 (segment (start 110.93 103.08) (end 107.33 103.08) (width 0.2) (layer "F.Cu") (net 13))
 (segment (start 104 99.75) (end 102.840001 99.75) (width 0.2) (layer "F.Cu") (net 13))
 (segment (start 102.840001 99.75) (end 102.54 99.449999) (width 0.2) (layer "F.Cu") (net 13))
 (segment (start 111.5 102.51) (end 110.93 103.08) (width 0.2) (layer "F.Cu") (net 13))
 (segment (start 107.33 103.08) (end 104 99.75) (width 0.2) (layer "F.Cu") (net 13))
 (segment (start 102.54 99.449999) (end 102.54 98.475) (width 0.2) (layer "F.Cu") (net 13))
 (segment (start 102.54 93.525) (end 102.54 94.499999) (width 0.2) (layer "F.Cu") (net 2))
 (segment (start 109.26 96) (end 110.75 97.49) (width 0.2) (layer "F.Cu") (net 2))
 (segment (start 104.040001 96) (end 109.26 96) (width 0.2) (layer "F.Cu") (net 2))
 (segment (start 102.54 94.499999) (end 104.040001 96) (width 0.2) (layer "F.Cu") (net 2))
 (segment (start 110.01 102.51) (end 104 96.5) (width 0.2) (layer "F.Cu") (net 3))
 (segment (start 103.270001 96.5) (end 101.27 94.499999) (width 0.2) (layer "F.Cu") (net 3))
 (segment (start 110.5 102.51) (end 110.01 102.51) (width 0.2) (layer "F.Cu") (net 3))
 (segment (start 101.27 94.499999) (end 101.27 93.525) (width 0.2) (layer "F.Cu") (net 3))
 (segment (start 104 96.5) (end 103.270001 96.5) (width 0.2) (layer "F.Cu") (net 3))
 (segment (start 104.5 105) (end 104.5 108.39) (width 0.2) (layer "F.Cu") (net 11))
 (segment (start 104.5 108.39) (end 104.6 108.49) (width 0.2) (layer "F.Cu") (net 11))
 (segment (start 101 101.106544) (end 100 100.106544) (width 0.2) (layer "F.Cu") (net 11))
 (segment (start 101.8875 102.3875) (end 104.5 105) (width 0.2) (layer "F.Cu") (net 11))
 (segment (start 100.975 102.275) (end 101 102.25) (width 0.2) (layer "F.Cu") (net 11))
 (segment (start 100.975 102.3875) (end 100.975 102.275) (width 0.2) (layer "F.Cu") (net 11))
 (segment (start 101 102.25) (end 101 101.106544) (width 0.2) (layer "F.Cu") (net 11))
 (segment (start 100.975 102.3875) (end 101.8875 102.3875) (width 0.2) (layer "F.Cu") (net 11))
 (segment (start 100 100.106544) (end 100 98.475) (width 0.2) (layer "F.Cu") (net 11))
 (segment (start 100.973496 105.973496) (end 98.776504 105.973496) (width 0.2) (layer "F.Cu") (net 23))
 (segment (start 98.776504 105.973496) (end 97.51 107.24) (width 0.2) (layer "F.Cu") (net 23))
 (segment (start 104.6 109.51) (end 106.8 107.31) (width 0.2) (layer "F.Cu") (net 23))
 (segment (start 101.6 109.5) (end 101.6 106.6) (width 0.2) (layer "F.Cu") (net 23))
 (segment (start 103.6 109.51) (end 103.31 109.8) (width 0.2) (layer "F.Cu") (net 23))
 (segment (start 101.6 106.6) (end 100.973496 105.973496) (width 0.2) (layer "F.Cu") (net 23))
 (segment (start 101.9 109.8) (end 101.6 109.5) (width 0.2) (layer "F.Cu") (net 23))
 (segment (start 103.31 109.8) (end 101.9 109.8) (width 0.2) (layer "F.Cu") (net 23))
 (segment (start 97.51 107.24) (end 97.5 107.24) (width 0.2) (layer "F.Cu") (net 23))
 (segment (start 106.8 107.31) (end 106.8 107.01) (width 0.2) (layer "F.Cu") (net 23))
 (segment (start 103.6 108.49) (end 103.11 108.49) (width 0.2) (layer "F.Cu") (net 12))
 (segment (start 100.325 104.315) (end 103.6 107.59) (width 0.2) (layer "F.Cu") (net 12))
 (segment (start 100.325 102.3875) (end 100.325 104.315) (width 0.2) (layer "F.Cu") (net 12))
 (segment (start 102.6 109) (end 102.4 109.2) (width 0.2) (layer "F.Cu") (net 12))
 (segment (start 105.1 105) (end 105.1 106.6) (width 0.2) (layer "F.Cu") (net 12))
 (segment (start 103.6 107.59) (end 103.6 108.49) (width 0.2) (layer "F.Cu") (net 12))
 (segment (start 101.4 101.3) (end 105.1 105) (width 0.2) (layer "F.Cu") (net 12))
 (segment (start 105.7 107.2) (end 105.7 107.5) (width 0.2) (layer "F.Cu") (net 12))
 (segment (start 101.4 98.605) (end 101.4 101.3) (width 0.2) (layer "F.Cu") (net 12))
 (segment (start 101.27 98.475) (end 101.4 98.605) (width 0.2) (layer "F.Cu") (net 12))
 (segment (start 105.1 106.6) (end 105.7 107.2) (width 0.2) (layer "F.Cu") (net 12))
 (segment (start 103.11 108.49) (end 102.6 109) (width 0.2) (layer "F.Cu") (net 12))
 (via (at 102.4 109.2) (size 0.6) (drill 0.3) (layers "F.Cu" "B.Cu") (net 12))
 (via (at 105.7 107.5) (size 0.6) (drill 0.3) (layers "F.Cu" "B.Cu") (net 12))
 (segment (start 104 109.2) (end 105.7 107.5) (width 0.2) (layer "B.Cu") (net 12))
 (segment (start 102.4 109.2) (end 104 109.2) (width 0.2) (layer "B.Cu") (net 12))
 (segment (start 98.8775 108.26) (end 99.025 108.1125) (width 0.2) (layer "F.Cu") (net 19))
 (segment (start 97.5 108.26) (end 98.8775 108.26) (width 0.2) (layer "F.Cu") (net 19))
 (segment (start 100 95.519448) (end 101.9 97.419448) (width 0.2) (layer "F.Cu") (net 4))
 (segment (start 106.8 105.99) (end 106.8 104.55) (width 0.2) (layer "F.Cu") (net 4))
 (segment (start 106.8 104.55) (end 101.9 99.65) (width 0.2) (layer "F.Cu") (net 4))
 (segment (start 101.9 97.419448) (end 101.9 99.65) (width 0.2) (layer "F.Cu") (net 4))
 (segment (start 100 93.525) (end 100 95.519448) (width 0.2) (layer "F.Cu") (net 4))
 (segment (start 99.85 91.75) (end 98.73 92.87) (width 0.2) (layer "F.Cu") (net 5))
 (segment (start 98.76 93.495) (end 98.73 93.525) (width 0.2) (layer "F.Cu") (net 5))
 (segment (start 99.35 101.325001) (end 99.675 101.650001) (width 0.2) (layer "F.Cu") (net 5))
 (segment (start 98.73 92.87) (end 98.73 93.525) (width 0.2) (layer "F.Cu") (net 5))
 (segment (start 99.675 101.650001) (end 99.675 102.3875) (width 0.2) (layer "F.Cu") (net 5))
 (segment (start 104.14 91.75) (end 99.85 91.75) (width 0.2) (layer "F.Cu") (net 5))
 (segment (start 98.73 93.525) (end 98.73 94.83) (width 0.2) (layer "F.Cu") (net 5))
 (segment (start 98.73 94.83) (end 99.35 95.45) (width 0.2) (layer "F.Cu") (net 5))
 (segment (start 99.35 96.25) (end 99.35 101.325001) (width 0.2) (layer "F.Cu") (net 5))
 (segment (start 99.35 95.45) (end 99.35 96.25) (width 0.2) (layer "F.Cu") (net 5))
 (segment (start 97.51 102.25) (end 98.8875 102.25) (width 0.2) (layer "F.Cu") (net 15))
 (segment (start 98.8875 102.25) (end 99.025 102.3875) (width 0.2) (layer "F.Cu") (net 15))
 (segment (start 96.9113 87.7387) (end 98.8387 87.7387) (width 0.2) (layer "F.Cu") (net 10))
 (segment (start 96.25 91.5) (end 96.25 88.4) (width 0.2) (layer "F.Cu") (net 10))
 (segment (start 98.1 97.845) (end 98.1 92.25) (width 0.2) (layer "F.Cu") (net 10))
 (segment (start 98.8387 87.7387) (end 99.2 88.1) (width 0.2) (layer "F.Cu") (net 10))
 (segment (start 99.2 88.1) (end 100.405 88.1) (width 0.2) (layer "F.Cu") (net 10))
 (segment (start 98.1 92.25) (end 97.85 92) (width 0.2) (layer "F.Cu") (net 10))
 (segment (start 96.25 88.4) (end 96.9113 87.7387) (width 0.2) (layer "F.Cu") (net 10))
 (segment (start 100.405 88.1) (end 101.27 88.965) (width 0.2) (layer "F.Cu") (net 10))
 (segment (start 96.75 92) (end 96.25 91.5) (width 0.2) (layer "F.Cu") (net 10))
 (segment (start 97.85 92) (end 96.75 92) (width 0.2) (layer "F.Cu") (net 10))
 (segment (start 98.73 98.475) (end 98.1 97.845) (width 0.2) (layer "F.Cu") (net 10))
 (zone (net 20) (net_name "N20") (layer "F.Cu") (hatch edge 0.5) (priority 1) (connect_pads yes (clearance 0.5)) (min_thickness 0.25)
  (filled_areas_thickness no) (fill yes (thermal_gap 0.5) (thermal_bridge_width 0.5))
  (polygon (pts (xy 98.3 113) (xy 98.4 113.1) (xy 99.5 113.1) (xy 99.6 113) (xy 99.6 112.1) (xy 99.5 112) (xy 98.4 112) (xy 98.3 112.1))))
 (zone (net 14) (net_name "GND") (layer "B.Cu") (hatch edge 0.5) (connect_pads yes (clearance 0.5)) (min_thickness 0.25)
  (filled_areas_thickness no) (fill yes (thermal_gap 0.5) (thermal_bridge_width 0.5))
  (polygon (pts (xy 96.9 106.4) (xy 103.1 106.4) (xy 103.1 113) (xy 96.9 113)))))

